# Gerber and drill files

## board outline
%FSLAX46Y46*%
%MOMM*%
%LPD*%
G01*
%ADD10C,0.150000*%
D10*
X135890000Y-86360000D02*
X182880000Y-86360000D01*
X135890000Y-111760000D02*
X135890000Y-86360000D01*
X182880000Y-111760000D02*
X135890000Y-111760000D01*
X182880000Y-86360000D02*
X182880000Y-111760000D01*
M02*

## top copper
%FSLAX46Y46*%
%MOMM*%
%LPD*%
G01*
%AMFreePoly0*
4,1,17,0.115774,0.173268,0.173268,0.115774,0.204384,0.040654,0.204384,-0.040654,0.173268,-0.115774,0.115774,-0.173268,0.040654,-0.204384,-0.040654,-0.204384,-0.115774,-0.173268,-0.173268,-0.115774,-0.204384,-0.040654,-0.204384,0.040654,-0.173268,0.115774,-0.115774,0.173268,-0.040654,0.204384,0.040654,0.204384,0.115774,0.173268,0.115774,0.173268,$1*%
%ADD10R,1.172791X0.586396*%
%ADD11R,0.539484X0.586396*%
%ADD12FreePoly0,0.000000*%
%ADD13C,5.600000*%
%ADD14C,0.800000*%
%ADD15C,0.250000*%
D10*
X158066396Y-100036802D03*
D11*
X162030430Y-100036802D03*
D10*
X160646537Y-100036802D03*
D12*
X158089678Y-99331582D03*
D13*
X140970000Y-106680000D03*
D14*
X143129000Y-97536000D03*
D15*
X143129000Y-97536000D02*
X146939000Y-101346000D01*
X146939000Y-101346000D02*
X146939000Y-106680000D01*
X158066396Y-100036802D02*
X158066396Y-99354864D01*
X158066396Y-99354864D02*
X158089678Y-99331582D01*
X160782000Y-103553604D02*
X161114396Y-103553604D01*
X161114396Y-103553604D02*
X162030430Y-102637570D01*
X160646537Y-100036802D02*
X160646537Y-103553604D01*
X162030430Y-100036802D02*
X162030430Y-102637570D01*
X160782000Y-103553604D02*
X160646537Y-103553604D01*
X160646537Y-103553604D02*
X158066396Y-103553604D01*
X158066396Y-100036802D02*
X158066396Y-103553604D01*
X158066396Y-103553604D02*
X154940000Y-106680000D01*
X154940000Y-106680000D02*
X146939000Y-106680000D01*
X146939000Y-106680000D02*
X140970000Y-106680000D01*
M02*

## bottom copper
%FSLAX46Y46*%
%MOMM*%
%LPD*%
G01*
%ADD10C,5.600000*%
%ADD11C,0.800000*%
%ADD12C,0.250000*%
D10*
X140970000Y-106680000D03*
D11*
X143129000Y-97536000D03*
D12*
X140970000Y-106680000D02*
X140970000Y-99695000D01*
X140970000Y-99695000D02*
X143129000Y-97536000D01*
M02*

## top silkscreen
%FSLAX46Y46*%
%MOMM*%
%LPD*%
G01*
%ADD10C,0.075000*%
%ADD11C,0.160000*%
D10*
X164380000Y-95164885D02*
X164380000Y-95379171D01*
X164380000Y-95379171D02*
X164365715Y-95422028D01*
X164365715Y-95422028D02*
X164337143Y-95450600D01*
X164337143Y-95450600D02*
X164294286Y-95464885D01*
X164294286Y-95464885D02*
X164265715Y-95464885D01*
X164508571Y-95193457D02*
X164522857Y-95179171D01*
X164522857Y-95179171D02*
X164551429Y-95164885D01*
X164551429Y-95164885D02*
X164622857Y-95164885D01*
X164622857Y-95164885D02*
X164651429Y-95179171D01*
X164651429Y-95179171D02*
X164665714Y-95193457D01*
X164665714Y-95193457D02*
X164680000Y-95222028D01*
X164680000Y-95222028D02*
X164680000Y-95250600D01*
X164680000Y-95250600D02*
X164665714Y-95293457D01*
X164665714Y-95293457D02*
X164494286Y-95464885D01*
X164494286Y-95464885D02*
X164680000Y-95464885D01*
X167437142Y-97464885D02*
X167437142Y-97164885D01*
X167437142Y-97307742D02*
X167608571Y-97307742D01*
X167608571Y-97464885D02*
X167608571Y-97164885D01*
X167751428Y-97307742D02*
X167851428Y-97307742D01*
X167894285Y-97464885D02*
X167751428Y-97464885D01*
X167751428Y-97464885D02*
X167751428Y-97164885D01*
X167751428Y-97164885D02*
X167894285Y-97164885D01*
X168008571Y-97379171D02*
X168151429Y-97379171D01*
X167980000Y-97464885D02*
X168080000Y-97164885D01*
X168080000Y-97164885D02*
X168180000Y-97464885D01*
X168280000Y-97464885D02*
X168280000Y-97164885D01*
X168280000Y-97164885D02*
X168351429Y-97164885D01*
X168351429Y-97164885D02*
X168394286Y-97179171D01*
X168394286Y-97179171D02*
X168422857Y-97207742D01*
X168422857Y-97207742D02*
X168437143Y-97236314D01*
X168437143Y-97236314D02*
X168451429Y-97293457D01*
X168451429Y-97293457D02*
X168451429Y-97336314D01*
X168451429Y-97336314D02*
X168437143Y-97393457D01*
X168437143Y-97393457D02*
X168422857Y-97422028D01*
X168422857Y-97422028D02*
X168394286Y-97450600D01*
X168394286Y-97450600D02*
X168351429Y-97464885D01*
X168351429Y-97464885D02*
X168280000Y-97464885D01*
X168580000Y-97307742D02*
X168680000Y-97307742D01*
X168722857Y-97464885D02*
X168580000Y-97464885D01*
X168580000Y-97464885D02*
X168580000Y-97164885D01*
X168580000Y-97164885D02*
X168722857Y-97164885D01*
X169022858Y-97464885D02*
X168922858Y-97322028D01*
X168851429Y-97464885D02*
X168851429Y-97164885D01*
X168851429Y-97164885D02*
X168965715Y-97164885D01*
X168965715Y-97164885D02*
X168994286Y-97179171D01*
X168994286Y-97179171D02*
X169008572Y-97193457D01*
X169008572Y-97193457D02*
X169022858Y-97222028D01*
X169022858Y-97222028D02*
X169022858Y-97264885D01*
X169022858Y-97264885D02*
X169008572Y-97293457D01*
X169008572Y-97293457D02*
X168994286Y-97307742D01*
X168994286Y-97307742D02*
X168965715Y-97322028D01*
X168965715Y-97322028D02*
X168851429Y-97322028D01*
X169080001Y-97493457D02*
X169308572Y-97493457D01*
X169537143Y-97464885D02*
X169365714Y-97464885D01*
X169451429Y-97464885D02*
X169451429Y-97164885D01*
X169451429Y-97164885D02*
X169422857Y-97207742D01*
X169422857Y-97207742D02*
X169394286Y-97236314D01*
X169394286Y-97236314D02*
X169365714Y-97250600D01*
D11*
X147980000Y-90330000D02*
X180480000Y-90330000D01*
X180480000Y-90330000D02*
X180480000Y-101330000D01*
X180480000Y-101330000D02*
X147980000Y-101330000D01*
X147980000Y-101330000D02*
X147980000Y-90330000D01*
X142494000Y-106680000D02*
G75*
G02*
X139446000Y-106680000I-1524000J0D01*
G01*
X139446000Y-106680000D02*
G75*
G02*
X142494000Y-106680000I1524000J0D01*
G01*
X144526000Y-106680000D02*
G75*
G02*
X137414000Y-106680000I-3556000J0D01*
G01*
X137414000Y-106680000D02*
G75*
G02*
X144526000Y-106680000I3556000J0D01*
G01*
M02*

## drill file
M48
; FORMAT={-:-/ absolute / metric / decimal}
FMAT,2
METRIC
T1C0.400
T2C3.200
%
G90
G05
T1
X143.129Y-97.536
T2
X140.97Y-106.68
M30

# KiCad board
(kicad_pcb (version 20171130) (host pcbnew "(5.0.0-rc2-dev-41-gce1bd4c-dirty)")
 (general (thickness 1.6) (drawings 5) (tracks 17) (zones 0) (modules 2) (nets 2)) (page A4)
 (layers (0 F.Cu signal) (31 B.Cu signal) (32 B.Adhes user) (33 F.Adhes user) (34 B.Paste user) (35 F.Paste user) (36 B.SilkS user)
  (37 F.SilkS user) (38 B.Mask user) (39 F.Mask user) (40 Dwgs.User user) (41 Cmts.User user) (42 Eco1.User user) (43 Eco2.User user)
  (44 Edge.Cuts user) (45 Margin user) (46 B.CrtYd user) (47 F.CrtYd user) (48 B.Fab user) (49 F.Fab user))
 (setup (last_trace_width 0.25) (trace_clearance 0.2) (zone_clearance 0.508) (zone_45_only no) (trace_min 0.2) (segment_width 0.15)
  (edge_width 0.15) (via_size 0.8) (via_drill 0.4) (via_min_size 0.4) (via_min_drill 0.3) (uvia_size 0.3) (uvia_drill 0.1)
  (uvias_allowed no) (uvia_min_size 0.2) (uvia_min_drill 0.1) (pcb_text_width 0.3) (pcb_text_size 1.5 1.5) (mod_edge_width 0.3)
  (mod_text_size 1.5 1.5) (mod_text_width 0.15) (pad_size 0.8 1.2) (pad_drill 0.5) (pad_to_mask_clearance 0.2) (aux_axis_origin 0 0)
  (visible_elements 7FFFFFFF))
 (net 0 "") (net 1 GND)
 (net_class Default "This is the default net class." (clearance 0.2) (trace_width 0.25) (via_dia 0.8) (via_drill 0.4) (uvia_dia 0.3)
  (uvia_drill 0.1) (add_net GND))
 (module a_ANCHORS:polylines (layer F.Cu) (at 157.48 100.33)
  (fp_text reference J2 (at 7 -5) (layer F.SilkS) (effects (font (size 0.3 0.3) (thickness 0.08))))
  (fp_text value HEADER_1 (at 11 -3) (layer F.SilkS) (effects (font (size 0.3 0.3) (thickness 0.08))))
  (fp_line (start -9.5 -10) (end 23 -10) (layer F.SilkS) (width 0.16))
  (fp_line (start 23 -10) (end 23 1) (layer F.SilkS) (width 0.16))
  (fp_line (start 23 1) (end -9.5 1) (layer F.SilkS) (width 0.16))
  (fp_line (start -9.5 1) (end -9.5 -10) (layer F.SilkS) (width 0.16))
  (pad 1 smd rect (at 0.586396 -0.293198) (size 1.172791 0.586396) (layers F.Cu F.Mask) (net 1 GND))
  (pad 1 smd rect (at 4.55043 -0.293198) (size 0.539484 0.586396) (layers F.Cu F.Mask) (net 1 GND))
  (pad 1 smd rect (at 3.166537 -0.293198) (size 1.172791 0.586396) (layers F.Cu F.Mask) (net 1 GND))
  (pad 1 smd custom (at 0.609678 -0.998418) (size 0.416776 0.416776) (layers F.Cu F.Mask) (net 1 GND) (zone_connect 0)
   (options (clearance outline) (anchor circle)) (primitives)))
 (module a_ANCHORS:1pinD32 (layer F.Cu) (at 140.97 106.68)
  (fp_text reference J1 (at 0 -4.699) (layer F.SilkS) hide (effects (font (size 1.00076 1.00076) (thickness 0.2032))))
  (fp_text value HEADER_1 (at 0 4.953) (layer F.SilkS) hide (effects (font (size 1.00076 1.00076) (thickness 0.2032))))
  (fp_circle (center 0 0) (end 0 1.524) (layer F.SilkS) (width 0.16))
  (fp_circle (center 0 0) (end 0 3.556) (layer F.SilkS) (width 0.16))
  (pad 1 thru_hole circle (at 0 0) (size 5.6 5.6) (drill 3.2004) (layers *.Cu *.Mask) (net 1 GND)))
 (gr_line (start 135.89 86.36) (end 182.88 86.36) (angle 90) (layer Edge.Cuts) (width 0.15))
 (gr_line (start 135.89 111.76) (end 135.89 86.36) (angle 90) (layer Edge.Cuts) (width 0.15))
 (gr_line (start 182.88 111.76) (end 135.89 111.76) (angle 90) (layer Edge.Cuts) (width 0.15))
 (gr_line (start 182.88 86.36) (end 182.88 111.76) (angle 90) (layer Edge.Cuts) (width 0.15))
 (segment (start 140.97 106.68) (end 140.97 99.695) (width 0.25) (layer B.Cu) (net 1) (status 400000))
 (segment (start 140.97 99.695) (end 143.129 97.536) (width 0.25) (layer B.Cu) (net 1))
 (via (at 143.129 97.536) (size 0.8) (drill 0.4) (layers F.Cu B.Cu) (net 1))
 (segment (start 143.129 97.536) (end 146.939 101.346) (width 0.25) (layer F.Cu) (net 1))
 (segment (start 146.939 101.346) (end 146.939 106.68) (width 0.25) (layer F.Cu) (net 1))
 (segment (start 158.066396 100.036802) (end 158.066396 99.354864) (width 0.25) (layer F.Cu) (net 1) (status C00000))
 (segment (start 158.066396 99.354864) (end 158.089678 99.331582) (width 0.25) (layer F.Cu) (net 1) (status C00000))
 (segment (start 160.782 103.553604) (end 161.114396 103.553604) (width 0.25) (layer F.Cu) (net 1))
 (segment (start 161.114396 103.553604) (end 162.03043 102.63757) (width 0.25) (layer F.Cu) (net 1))
 (segment (start 160.646537 100.036802) (end 160.646537 103.553604) (width 0.25) (layer F.Cu) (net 1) (status 400000))
 (segment (start 162.03043 100.036802) (end 162.03043 102.63757) (width 0.25) (layer F.Cu) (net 1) (status 400000))
 (segment (start 160.782 103.553604) (end 160.646537 103.553604) (width 0.25) (layer F.Cu) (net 1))
 (segment (start 160.646537 103.553604) (end 158.066396 103.553604) (width 0.25) (layer F.Cu) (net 1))
 (segment (start 158.066396 100.036802) (end 158.066396 103.553604) (width 0.25) (layer F.Cu) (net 1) (status 400000))
 (segment (start 158.066396 103.553604) (end 154.94 106.68) (width 0.25) (layer F.Cu) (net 1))
 (segment (start 154.94 106.68) (end 146.939 106.68) (width 0.25) (layer F.Cu) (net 1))
 (segment (start 146.939 106.68) (end 140.97 106.68) (width 0.25) (layer F.Cu) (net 1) (status 800000)))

